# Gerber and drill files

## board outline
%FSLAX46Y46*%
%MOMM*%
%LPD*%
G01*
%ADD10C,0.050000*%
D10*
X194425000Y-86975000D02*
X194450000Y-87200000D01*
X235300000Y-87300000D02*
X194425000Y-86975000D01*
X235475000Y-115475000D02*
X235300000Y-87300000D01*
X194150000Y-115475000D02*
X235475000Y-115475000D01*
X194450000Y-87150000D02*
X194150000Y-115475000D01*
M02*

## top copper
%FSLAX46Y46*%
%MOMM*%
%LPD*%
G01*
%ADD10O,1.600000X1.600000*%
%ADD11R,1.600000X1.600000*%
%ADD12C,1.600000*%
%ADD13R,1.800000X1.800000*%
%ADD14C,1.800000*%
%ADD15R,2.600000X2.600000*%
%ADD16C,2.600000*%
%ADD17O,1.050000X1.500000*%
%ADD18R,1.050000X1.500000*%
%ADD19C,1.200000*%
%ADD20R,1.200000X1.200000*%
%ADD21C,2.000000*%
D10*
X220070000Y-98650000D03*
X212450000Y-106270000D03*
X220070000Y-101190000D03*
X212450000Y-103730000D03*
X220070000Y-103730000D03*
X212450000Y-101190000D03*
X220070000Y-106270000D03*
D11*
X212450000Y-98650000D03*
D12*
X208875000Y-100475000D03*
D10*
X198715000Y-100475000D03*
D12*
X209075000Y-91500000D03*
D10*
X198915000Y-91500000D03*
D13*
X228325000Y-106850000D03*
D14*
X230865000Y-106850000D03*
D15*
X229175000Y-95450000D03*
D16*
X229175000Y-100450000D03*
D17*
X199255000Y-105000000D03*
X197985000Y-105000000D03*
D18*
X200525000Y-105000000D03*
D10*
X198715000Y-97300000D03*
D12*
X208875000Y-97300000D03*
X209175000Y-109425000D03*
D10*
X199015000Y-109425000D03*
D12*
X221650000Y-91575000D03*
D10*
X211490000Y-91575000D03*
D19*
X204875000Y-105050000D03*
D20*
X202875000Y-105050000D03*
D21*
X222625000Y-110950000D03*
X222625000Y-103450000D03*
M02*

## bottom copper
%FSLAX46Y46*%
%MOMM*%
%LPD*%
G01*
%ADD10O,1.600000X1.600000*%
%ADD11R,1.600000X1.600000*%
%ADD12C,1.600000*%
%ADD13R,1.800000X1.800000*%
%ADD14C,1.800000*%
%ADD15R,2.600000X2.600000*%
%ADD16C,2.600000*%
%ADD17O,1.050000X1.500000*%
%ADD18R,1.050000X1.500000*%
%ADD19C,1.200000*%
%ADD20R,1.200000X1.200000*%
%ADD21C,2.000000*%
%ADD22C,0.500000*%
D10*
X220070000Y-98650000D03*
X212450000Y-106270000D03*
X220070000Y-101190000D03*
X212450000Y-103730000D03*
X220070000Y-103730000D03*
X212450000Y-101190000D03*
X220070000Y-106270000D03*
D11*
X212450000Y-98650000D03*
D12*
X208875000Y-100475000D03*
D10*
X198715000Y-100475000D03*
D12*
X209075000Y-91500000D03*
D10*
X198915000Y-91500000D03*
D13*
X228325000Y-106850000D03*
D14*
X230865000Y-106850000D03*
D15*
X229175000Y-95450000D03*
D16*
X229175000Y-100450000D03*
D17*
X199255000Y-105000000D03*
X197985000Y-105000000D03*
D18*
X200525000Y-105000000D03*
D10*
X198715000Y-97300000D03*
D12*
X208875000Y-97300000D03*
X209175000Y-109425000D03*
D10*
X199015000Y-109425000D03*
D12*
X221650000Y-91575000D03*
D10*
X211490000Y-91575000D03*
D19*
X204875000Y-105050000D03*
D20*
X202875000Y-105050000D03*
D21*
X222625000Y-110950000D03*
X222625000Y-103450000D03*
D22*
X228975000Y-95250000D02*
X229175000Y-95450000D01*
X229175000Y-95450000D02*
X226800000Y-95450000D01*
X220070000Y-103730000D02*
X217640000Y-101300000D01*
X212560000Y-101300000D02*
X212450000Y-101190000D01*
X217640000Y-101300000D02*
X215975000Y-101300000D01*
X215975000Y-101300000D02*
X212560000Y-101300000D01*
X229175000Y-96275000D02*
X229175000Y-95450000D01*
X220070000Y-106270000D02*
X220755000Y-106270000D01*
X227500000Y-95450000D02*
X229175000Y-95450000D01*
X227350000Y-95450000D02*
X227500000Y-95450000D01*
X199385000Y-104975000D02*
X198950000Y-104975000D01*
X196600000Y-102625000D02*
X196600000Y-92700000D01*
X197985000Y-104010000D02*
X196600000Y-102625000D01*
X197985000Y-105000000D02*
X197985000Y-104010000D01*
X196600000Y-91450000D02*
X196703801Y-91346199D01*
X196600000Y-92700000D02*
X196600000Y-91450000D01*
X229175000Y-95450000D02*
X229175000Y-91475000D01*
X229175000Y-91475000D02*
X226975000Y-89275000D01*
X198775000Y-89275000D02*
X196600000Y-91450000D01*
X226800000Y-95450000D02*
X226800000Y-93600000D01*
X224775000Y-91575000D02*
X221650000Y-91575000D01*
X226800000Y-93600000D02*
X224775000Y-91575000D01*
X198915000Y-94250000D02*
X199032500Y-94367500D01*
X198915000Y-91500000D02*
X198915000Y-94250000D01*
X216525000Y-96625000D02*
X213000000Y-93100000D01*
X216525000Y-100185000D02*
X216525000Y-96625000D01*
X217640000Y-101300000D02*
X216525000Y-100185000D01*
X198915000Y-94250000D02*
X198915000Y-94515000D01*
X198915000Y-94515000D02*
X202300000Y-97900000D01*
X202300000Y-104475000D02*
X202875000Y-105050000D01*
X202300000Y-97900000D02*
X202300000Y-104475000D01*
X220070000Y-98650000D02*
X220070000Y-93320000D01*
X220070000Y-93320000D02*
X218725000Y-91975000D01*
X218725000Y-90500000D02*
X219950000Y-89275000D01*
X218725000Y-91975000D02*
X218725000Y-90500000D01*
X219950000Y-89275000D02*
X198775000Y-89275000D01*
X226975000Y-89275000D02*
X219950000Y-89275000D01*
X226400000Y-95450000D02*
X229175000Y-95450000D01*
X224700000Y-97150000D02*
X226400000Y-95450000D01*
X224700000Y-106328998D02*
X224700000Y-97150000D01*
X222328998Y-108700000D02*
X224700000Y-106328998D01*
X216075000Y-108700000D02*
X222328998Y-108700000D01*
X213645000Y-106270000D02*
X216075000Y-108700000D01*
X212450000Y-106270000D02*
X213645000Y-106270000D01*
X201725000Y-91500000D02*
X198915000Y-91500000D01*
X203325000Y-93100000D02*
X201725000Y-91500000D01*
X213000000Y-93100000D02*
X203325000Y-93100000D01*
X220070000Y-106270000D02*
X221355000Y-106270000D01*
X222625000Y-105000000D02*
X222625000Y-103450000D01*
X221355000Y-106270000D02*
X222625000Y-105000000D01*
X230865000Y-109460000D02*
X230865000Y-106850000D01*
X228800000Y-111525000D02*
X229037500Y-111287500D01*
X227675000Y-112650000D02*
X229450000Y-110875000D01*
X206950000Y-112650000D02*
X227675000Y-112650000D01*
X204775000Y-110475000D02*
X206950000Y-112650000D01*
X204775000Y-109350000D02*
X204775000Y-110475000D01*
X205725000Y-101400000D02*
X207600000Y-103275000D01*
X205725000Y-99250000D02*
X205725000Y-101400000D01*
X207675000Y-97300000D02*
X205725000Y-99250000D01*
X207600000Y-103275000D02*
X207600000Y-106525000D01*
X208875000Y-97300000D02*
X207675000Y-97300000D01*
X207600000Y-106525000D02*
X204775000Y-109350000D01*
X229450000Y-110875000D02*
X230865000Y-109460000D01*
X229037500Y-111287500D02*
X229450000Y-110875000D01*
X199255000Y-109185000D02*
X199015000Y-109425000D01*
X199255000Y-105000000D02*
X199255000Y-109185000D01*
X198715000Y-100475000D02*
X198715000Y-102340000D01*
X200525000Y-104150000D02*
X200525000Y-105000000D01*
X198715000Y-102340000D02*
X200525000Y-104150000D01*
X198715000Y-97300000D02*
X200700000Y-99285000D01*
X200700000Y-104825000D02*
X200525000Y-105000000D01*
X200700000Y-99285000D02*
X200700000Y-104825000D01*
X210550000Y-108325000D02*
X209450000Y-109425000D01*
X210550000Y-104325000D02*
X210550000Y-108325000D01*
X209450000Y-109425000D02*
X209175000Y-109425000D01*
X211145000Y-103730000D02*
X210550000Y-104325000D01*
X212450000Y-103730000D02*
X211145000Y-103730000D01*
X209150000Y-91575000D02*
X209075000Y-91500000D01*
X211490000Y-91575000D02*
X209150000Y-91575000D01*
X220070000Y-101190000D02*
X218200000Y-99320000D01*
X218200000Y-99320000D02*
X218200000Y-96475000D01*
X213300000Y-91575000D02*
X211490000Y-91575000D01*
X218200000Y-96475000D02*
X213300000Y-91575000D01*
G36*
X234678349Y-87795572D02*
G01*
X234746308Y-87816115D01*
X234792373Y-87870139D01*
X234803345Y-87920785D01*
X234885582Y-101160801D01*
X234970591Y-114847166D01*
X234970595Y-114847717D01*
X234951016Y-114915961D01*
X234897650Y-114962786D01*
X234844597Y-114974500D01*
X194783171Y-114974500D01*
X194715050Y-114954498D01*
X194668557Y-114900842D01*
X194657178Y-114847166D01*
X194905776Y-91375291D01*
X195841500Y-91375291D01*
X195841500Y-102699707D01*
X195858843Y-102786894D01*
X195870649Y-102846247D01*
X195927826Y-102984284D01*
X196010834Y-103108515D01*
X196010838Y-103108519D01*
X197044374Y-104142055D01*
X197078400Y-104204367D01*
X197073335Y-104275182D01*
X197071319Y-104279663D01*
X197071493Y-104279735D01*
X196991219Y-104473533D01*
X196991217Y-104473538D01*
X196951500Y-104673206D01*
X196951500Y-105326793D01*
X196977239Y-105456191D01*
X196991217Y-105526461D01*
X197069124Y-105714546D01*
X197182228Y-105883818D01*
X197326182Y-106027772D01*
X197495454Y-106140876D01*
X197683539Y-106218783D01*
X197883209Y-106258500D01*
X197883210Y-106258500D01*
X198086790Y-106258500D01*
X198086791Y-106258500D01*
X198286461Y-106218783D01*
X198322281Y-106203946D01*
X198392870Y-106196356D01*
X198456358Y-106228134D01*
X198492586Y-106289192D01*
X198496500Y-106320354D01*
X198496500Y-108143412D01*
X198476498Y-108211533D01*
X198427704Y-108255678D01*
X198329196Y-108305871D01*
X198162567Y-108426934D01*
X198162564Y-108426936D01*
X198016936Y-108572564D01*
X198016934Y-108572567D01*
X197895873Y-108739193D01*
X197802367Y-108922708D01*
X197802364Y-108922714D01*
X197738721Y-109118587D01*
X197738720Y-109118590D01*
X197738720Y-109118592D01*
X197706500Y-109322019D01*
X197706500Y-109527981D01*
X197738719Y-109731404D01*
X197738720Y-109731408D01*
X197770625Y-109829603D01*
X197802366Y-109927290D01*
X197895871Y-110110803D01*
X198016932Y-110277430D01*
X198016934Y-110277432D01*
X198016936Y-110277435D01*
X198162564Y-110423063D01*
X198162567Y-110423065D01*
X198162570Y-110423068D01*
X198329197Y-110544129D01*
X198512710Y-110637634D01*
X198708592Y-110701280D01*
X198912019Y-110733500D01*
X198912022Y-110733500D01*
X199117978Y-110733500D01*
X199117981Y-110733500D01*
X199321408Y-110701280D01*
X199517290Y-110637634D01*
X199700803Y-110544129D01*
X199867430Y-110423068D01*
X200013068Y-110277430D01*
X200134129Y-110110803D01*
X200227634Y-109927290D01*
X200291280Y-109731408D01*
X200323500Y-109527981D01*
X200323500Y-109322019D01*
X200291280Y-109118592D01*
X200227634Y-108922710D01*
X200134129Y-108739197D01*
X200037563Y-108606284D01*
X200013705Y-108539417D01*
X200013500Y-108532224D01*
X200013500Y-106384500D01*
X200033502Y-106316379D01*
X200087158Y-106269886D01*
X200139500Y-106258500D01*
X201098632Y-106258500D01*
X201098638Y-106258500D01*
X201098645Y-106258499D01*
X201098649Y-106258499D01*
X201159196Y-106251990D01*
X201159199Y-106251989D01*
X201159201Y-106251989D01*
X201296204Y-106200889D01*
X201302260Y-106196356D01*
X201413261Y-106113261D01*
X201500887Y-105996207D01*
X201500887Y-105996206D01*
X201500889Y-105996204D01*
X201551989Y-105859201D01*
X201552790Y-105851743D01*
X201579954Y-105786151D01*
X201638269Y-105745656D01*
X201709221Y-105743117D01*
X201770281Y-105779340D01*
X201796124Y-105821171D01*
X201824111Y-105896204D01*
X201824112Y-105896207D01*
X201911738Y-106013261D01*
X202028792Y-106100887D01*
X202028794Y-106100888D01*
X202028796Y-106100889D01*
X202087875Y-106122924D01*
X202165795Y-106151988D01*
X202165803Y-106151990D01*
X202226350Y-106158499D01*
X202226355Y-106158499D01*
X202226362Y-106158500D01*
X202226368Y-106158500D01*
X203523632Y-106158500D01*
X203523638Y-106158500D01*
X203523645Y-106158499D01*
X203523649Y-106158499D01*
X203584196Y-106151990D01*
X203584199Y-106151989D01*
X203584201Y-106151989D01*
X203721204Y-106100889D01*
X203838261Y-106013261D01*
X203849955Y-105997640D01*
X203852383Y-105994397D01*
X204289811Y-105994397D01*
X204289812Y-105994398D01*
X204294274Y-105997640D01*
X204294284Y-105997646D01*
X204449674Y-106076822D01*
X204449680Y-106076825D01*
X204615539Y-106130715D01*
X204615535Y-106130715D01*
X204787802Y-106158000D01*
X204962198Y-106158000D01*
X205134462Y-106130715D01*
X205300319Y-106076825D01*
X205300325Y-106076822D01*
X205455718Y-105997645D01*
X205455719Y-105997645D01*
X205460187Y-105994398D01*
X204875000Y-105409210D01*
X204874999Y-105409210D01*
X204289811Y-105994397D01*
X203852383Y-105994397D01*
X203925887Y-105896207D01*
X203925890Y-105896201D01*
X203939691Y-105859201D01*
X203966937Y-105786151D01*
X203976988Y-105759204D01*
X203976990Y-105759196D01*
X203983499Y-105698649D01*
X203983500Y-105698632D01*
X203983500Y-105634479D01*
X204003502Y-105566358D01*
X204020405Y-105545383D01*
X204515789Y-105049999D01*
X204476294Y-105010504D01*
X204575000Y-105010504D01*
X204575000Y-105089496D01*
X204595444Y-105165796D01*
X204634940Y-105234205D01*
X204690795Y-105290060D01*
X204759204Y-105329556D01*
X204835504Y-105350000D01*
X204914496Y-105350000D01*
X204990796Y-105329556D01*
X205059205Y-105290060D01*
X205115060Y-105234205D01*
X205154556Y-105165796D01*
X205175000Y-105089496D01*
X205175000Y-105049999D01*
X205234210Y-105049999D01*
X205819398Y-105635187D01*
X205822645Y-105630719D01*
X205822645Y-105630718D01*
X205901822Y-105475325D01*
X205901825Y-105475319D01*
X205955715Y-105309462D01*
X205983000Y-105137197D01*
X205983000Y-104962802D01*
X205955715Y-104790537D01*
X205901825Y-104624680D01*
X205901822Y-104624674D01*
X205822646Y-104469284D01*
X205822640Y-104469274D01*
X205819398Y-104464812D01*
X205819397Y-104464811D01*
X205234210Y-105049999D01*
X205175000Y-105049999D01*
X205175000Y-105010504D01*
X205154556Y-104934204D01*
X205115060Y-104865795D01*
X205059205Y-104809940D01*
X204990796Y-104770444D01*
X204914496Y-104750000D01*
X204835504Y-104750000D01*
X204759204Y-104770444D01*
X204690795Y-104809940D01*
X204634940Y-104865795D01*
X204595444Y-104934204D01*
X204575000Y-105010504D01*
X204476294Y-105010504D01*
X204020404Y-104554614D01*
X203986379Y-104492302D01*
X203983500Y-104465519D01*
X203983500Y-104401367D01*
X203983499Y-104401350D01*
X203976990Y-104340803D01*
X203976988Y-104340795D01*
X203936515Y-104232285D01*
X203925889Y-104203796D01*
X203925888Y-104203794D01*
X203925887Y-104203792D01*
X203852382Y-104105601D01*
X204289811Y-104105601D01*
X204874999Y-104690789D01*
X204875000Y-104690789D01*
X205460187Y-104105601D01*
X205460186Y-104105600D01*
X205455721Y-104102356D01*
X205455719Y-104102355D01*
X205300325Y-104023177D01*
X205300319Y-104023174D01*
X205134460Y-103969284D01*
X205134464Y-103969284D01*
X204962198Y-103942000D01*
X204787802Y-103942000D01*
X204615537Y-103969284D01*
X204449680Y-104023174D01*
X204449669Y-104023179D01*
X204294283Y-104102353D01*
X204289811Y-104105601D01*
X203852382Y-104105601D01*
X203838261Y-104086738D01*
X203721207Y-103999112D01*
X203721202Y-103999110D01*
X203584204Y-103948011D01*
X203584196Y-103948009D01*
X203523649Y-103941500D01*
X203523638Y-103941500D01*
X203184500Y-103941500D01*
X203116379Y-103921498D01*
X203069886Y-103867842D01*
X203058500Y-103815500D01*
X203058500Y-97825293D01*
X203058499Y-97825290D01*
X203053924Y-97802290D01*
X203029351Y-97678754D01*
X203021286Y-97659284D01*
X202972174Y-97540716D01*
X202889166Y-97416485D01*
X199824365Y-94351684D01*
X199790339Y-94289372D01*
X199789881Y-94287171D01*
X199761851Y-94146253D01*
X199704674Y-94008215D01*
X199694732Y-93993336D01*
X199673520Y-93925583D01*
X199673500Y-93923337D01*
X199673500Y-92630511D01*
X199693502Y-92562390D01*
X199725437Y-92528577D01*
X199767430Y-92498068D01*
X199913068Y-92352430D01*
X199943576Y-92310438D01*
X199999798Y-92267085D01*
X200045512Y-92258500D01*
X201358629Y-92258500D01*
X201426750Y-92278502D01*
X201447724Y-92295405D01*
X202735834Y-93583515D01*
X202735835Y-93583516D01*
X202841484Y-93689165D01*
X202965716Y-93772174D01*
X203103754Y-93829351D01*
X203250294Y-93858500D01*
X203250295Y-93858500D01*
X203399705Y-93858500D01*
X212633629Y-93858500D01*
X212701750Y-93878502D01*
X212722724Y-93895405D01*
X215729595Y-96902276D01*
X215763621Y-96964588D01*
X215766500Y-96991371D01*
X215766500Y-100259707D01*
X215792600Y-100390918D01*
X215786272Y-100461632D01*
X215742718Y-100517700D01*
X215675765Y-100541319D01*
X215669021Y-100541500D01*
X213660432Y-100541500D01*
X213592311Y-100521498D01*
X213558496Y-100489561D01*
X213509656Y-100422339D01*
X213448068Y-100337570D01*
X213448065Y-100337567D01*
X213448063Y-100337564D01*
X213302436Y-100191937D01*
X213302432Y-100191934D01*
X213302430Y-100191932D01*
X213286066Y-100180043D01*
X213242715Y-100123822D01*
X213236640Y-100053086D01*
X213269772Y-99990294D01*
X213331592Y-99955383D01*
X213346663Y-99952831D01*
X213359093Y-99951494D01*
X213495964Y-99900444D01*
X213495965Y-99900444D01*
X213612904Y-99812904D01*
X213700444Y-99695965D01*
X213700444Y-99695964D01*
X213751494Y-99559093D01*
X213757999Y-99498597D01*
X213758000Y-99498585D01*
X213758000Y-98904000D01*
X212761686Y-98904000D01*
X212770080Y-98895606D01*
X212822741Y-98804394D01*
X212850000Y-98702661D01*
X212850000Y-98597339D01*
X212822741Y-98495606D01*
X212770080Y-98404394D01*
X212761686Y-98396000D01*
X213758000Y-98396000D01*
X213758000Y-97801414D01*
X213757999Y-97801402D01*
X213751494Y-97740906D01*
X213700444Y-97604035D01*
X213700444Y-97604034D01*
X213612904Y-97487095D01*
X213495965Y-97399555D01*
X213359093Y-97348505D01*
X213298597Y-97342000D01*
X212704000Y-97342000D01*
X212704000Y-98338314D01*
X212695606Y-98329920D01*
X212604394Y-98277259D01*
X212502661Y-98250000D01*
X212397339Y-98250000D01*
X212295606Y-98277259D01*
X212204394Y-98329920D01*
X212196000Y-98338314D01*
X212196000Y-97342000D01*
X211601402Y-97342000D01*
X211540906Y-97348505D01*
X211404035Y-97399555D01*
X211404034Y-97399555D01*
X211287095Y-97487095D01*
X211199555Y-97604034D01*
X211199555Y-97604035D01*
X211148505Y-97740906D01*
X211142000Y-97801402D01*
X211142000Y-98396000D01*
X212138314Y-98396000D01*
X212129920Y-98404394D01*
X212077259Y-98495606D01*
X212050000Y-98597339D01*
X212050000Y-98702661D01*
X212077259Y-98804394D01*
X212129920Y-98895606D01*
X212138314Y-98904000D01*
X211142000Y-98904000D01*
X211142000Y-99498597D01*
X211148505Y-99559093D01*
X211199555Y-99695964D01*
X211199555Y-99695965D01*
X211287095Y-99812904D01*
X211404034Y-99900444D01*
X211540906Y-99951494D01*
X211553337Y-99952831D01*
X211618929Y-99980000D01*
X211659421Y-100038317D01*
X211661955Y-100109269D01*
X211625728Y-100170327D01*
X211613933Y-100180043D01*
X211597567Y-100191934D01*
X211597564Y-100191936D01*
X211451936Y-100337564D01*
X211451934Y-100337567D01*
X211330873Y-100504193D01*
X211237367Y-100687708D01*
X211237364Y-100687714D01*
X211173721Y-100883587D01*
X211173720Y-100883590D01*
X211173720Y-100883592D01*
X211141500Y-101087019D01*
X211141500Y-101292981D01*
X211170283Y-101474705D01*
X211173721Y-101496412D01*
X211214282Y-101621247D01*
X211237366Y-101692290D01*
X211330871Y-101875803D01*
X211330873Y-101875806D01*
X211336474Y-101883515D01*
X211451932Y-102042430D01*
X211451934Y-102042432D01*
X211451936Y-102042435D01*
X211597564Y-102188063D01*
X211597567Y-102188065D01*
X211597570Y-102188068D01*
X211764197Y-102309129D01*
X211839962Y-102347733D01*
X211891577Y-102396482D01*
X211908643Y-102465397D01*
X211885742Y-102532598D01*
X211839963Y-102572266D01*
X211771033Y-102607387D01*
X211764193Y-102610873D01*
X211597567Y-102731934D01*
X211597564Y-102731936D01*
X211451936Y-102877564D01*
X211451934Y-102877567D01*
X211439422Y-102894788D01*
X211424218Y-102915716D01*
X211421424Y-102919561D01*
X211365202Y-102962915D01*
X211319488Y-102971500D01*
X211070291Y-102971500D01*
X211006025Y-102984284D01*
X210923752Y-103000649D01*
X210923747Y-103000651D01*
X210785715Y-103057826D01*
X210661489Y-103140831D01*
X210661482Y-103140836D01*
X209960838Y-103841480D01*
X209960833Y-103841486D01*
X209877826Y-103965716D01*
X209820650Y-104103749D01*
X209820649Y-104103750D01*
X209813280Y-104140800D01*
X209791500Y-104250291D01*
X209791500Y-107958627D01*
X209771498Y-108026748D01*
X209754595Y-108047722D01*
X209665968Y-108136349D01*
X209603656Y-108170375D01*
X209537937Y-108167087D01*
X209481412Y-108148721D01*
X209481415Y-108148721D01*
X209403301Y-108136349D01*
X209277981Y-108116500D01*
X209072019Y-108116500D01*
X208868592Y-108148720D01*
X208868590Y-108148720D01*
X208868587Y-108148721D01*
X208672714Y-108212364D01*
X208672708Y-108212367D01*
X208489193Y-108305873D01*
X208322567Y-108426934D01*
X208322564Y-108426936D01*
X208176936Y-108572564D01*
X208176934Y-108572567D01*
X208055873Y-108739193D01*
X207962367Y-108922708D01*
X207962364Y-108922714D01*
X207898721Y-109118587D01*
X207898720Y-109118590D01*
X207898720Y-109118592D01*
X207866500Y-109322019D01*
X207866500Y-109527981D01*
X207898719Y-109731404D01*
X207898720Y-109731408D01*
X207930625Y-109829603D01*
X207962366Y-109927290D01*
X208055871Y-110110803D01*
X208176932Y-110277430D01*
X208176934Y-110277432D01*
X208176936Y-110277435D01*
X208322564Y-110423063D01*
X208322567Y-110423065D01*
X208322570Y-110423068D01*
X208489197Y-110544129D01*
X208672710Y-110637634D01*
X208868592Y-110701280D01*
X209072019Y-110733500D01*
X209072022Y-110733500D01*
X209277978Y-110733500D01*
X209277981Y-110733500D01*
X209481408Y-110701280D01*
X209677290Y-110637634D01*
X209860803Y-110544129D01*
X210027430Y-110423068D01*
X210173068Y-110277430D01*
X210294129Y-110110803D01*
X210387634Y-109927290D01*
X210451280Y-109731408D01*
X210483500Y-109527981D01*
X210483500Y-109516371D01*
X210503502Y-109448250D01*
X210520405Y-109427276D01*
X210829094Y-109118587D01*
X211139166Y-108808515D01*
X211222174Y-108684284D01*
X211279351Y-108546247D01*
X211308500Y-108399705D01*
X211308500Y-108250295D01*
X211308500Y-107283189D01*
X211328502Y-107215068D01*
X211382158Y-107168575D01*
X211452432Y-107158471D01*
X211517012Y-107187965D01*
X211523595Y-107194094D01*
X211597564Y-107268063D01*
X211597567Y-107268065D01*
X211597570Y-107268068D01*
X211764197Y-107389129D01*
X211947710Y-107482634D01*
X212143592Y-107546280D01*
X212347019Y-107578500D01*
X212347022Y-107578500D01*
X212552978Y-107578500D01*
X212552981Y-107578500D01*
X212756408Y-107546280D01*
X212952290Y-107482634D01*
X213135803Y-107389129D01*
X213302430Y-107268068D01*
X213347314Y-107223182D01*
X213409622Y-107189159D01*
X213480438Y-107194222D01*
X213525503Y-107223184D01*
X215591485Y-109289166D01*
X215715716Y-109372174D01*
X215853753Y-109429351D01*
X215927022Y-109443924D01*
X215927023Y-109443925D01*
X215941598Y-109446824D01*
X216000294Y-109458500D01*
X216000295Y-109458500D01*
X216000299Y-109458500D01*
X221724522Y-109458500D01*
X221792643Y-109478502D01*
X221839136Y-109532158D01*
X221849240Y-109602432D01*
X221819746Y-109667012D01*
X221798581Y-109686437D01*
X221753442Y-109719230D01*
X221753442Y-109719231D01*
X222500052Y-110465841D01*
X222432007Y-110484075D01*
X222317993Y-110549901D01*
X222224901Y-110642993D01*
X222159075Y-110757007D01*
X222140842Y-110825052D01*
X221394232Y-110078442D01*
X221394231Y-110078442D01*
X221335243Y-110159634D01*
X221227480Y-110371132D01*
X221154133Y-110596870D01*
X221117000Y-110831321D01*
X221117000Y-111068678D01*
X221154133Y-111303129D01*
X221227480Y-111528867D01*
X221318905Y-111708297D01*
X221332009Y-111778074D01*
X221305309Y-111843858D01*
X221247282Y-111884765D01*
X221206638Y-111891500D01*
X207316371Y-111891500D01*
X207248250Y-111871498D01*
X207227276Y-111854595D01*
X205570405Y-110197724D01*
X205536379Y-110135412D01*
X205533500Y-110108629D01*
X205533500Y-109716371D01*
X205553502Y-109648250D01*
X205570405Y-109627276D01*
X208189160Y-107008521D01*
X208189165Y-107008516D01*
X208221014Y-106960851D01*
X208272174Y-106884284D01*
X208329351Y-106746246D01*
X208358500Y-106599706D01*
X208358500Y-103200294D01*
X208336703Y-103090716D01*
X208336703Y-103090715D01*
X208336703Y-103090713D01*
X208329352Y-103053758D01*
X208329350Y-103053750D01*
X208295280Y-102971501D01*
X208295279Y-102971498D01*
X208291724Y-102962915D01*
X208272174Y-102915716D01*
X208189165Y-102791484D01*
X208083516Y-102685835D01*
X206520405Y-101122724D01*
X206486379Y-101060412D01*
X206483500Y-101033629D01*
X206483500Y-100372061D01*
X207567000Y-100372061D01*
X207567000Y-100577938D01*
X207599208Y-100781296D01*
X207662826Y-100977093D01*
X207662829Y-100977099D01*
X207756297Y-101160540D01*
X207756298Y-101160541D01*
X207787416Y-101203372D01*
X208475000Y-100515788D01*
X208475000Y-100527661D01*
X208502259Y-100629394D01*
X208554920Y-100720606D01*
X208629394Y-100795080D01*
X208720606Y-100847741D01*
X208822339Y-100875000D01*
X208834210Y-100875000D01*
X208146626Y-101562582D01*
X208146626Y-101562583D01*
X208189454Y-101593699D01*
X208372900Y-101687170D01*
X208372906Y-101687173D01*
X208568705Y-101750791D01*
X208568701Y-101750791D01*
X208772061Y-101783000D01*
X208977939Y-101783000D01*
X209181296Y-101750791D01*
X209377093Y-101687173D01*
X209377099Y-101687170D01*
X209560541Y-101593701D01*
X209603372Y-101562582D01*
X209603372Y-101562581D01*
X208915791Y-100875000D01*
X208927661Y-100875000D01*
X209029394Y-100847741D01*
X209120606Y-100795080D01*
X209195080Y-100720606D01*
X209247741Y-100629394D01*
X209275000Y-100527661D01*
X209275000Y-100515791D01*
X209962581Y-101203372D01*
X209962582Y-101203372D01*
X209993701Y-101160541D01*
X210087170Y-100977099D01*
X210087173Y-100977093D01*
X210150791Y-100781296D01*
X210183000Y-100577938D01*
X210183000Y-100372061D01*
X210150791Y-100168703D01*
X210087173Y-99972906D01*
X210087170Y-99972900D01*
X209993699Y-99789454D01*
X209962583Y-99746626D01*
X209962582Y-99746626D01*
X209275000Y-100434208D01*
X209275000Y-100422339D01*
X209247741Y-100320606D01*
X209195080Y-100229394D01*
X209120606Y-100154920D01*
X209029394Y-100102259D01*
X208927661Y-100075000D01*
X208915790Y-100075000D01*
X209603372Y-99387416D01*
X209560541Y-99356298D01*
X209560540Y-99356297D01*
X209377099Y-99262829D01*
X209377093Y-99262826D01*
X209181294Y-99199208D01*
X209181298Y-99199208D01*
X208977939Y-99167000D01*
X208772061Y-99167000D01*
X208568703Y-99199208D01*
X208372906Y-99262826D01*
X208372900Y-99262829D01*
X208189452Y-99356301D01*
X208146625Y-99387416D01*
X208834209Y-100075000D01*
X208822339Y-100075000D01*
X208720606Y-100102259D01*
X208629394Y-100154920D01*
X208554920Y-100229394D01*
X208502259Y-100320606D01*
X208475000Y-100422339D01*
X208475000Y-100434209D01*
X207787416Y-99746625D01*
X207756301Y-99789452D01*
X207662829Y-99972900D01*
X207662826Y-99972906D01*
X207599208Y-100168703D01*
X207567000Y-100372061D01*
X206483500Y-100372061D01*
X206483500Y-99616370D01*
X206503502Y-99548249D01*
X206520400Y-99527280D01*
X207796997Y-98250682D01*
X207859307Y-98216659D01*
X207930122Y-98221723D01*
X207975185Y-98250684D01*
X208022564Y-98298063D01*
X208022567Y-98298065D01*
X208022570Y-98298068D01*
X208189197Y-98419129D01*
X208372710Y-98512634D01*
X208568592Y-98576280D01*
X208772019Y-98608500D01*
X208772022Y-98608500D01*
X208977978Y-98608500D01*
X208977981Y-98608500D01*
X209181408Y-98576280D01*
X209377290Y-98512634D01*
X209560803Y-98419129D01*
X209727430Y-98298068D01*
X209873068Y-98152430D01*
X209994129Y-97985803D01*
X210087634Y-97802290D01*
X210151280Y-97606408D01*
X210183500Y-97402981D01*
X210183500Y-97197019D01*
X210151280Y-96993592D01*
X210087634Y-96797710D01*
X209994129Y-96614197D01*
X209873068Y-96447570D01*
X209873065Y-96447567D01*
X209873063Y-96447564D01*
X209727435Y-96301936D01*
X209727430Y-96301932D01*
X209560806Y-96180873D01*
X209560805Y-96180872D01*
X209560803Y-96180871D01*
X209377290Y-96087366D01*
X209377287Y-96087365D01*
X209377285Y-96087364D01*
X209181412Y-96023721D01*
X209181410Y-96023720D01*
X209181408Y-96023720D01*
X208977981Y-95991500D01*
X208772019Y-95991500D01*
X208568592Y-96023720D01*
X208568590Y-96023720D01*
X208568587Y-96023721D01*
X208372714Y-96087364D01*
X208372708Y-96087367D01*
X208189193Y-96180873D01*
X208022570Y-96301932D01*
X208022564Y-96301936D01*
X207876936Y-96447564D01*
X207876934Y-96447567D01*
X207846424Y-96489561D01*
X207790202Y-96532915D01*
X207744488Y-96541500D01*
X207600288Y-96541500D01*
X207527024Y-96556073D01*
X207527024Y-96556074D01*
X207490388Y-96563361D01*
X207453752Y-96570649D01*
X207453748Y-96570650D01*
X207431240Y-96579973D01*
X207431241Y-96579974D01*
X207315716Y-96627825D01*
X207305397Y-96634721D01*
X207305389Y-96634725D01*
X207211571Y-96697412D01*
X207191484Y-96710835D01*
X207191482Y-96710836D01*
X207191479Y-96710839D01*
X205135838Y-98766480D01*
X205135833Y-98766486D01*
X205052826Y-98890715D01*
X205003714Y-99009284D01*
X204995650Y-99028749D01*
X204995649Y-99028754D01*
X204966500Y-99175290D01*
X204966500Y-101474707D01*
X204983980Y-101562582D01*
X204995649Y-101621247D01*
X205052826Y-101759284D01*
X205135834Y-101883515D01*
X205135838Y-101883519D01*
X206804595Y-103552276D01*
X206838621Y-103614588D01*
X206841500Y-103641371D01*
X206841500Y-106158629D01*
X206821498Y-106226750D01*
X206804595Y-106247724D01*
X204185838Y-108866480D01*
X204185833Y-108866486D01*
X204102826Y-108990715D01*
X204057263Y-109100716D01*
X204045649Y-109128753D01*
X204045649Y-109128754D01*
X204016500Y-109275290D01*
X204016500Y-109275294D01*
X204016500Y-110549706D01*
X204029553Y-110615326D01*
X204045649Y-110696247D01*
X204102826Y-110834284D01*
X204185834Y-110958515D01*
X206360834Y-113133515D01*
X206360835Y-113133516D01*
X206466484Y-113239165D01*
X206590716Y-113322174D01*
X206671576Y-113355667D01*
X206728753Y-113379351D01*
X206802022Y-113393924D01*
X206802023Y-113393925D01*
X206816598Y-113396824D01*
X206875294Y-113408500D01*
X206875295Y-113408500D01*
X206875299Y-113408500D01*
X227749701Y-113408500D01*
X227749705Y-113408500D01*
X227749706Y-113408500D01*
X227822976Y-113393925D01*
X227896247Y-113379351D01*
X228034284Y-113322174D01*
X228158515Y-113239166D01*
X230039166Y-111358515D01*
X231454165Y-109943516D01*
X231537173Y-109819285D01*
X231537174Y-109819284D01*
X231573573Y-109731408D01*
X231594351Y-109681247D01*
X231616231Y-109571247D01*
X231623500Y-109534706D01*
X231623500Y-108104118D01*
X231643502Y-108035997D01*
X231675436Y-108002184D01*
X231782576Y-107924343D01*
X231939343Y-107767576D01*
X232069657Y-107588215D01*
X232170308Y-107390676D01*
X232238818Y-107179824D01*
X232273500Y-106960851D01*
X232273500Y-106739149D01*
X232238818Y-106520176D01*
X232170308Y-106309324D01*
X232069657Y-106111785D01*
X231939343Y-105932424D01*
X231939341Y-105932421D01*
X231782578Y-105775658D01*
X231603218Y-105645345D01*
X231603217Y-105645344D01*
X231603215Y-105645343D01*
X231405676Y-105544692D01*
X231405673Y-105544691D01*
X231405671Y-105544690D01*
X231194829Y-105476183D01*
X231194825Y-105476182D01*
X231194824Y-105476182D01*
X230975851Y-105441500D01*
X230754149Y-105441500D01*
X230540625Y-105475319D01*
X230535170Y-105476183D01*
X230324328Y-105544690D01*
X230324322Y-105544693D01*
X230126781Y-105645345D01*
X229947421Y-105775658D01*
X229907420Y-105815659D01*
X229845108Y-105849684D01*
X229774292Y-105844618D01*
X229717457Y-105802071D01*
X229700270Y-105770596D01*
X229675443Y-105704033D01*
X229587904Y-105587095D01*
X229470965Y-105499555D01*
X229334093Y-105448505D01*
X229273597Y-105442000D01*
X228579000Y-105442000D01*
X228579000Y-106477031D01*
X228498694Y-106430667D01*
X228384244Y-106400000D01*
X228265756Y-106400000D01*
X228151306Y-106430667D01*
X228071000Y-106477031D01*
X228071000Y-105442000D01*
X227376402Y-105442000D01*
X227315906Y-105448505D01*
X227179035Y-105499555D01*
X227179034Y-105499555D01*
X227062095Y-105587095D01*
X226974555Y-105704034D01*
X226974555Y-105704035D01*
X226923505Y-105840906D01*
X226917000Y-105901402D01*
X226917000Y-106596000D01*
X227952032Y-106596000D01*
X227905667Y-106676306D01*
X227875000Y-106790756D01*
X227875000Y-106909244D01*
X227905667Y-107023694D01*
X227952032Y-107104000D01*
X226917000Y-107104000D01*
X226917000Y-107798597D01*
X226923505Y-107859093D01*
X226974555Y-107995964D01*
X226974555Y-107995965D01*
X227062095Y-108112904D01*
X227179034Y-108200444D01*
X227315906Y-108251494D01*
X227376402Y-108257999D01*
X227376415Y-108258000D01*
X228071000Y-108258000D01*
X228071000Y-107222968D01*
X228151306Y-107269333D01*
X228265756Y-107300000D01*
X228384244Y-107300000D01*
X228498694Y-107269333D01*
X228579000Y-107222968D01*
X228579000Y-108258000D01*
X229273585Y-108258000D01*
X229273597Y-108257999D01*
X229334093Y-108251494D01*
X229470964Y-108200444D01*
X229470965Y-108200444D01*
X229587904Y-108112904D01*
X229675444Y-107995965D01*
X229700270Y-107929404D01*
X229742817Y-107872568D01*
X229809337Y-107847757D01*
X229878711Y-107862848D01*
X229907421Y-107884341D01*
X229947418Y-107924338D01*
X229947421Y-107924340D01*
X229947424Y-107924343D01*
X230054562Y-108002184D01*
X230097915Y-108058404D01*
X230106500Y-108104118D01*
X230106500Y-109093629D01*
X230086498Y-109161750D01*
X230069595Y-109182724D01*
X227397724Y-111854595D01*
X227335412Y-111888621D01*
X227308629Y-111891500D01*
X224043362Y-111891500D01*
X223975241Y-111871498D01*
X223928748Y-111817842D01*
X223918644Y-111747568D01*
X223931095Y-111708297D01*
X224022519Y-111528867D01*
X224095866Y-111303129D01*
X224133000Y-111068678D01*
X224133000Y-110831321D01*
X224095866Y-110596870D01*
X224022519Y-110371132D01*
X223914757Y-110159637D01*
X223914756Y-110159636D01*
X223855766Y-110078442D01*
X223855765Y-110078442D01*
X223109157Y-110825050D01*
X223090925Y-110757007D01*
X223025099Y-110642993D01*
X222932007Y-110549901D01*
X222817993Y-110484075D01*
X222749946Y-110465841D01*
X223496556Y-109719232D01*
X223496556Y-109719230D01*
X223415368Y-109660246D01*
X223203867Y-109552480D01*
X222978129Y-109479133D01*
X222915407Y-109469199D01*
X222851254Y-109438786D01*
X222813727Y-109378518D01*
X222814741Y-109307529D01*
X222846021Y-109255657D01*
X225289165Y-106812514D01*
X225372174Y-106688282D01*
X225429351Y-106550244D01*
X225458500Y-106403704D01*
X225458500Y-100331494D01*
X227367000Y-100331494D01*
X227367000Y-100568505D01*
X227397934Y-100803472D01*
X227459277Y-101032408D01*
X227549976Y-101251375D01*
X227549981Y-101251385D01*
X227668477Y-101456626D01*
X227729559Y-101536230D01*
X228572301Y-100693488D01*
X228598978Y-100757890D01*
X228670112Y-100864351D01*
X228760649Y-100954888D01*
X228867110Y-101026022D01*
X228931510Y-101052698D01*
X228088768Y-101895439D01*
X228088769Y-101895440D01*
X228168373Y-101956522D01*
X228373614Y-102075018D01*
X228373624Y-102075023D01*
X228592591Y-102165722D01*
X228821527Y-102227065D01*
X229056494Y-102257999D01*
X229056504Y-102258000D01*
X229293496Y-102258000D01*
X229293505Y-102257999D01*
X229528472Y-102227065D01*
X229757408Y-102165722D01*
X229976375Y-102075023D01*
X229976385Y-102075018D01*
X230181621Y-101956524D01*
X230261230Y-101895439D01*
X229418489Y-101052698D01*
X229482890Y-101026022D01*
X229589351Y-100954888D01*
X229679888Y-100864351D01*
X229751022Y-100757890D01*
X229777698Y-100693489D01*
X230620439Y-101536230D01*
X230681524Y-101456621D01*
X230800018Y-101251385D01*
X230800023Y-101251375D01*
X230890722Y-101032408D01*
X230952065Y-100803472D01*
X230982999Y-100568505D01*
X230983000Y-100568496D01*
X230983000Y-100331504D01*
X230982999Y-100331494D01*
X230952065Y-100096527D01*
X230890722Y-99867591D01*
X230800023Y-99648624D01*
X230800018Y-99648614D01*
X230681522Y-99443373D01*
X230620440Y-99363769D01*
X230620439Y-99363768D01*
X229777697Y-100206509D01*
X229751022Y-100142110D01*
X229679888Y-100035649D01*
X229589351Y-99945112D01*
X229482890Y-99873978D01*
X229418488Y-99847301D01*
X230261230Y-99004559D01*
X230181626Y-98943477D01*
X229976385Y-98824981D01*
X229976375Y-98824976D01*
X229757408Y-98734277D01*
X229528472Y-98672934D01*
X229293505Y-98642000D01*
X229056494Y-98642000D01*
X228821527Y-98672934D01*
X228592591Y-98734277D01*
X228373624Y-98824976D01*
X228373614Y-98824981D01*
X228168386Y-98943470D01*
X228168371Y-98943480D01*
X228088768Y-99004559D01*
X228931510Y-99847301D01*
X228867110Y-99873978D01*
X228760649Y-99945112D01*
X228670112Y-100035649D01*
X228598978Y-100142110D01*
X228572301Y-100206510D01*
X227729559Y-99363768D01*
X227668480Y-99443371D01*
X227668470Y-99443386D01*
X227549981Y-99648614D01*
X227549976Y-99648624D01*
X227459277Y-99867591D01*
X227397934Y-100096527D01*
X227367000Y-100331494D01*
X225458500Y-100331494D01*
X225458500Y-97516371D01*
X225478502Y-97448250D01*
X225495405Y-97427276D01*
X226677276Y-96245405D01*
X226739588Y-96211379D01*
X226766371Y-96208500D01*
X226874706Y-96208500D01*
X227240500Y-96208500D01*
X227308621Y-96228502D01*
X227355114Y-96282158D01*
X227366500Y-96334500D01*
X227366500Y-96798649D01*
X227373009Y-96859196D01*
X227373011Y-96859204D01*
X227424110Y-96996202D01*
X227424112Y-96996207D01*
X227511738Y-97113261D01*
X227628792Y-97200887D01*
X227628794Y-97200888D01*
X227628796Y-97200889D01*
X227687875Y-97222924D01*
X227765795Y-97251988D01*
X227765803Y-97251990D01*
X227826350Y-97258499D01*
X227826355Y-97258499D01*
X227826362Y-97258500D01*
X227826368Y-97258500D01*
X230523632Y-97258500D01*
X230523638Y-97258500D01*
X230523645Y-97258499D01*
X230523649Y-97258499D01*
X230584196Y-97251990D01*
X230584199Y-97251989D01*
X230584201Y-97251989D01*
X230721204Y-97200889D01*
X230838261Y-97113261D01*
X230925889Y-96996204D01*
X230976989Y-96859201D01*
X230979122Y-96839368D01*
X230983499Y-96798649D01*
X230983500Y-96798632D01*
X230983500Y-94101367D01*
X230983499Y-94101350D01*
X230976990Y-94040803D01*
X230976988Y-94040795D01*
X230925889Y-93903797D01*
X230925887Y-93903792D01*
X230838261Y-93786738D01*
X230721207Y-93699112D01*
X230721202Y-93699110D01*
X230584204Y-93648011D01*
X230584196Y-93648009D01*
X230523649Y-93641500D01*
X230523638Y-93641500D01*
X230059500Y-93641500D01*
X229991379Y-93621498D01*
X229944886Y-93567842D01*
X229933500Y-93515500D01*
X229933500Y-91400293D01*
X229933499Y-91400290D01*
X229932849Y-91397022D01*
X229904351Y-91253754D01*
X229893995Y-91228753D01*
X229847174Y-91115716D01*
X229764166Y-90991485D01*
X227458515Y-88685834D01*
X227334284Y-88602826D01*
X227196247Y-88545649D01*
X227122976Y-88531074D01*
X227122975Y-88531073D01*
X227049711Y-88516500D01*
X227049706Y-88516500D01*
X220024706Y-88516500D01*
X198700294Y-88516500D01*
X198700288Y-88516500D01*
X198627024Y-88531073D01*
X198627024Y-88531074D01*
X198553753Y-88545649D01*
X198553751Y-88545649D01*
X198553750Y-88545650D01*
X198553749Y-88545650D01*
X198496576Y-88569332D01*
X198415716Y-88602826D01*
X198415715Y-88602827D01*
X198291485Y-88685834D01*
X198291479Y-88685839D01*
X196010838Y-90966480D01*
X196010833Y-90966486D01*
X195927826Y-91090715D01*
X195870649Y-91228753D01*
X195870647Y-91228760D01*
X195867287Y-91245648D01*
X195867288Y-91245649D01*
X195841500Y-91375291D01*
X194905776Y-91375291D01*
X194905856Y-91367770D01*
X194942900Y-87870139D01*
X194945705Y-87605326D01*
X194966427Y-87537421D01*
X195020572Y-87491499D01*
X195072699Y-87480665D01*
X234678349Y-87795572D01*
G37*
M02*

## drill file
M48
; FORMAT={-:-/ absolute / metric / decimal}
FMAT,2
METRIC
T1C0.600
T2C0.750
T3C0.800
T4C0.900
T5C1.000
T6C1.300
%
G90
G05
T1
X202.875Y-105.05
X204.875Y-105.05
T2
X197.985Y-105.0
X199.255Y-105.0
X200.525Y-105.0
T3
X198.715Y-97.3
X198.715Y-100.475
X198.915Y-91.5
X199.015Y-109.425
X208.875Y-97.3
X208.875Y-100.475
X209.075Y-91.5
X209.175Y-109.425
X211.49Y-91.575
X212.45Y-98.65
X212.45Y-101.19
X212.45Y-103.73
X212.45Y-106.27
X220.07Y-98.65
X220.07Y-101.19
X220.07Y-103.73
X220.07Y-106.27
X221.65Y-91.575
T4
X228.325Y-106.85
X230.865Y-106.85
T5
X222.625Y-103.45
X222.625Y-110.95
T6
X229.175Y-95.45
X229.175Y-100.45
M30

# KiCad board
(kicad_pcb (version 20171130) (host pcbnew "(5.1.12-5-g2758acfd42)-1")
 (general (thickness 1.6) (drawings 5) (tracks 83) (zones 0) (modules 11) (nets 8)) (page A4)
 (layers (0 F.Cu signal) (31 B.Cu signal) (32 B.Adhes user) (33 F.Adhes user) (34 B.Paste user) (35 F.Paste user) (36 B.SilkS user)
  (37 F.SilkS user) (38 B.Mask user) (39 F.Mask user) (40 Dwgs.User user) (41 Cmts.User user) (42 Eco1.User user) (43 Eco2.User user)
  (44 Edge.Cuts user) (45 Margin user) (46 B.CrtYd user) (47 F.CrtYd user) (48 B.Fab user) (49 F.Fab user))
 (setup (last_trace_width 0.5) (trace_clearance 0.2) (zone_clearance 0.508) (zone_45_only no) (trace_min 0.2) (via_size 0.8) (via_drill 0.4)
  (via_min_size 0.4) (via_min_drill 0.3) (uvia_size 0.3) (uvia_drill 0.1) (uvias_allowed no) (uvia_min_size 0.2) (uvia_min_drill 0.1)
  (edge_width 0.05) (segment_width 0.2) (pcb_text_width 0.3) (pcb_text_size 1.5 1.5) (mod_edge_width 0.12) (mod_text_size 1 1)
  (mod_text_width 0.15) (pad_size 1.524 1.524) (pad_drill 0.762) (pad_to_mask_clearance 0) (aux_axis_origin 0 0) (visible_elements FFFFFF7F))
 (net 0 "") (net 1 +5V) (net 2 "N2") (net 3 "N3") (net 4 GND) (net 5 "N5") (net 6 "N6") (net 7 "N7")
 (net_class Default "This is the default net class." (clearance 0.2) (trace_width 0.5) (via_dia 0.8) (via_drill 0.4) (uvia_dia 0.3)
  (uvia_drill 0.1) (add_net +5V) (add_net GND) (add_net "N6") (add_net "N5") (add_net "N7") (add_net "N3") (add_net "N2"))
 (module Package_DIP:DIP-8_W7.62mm (layer F.Cu) (at 212.45 98.65)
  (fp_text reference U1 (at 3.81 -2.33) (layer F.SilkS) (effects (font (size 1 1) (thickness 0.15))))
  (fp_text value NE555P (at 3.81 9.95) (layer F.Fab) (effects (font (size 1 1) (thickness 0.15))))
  (pad 8 thru_hole oval (at 7.62 0) (size 1.6 1.6) (drill 0.8) (layers *.Cu *.Mask) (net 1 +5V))
  (pad 4 thru_hole oval (at 0 7.62) (size 1.6 1.6) (drill 0.8) (layers *.Cu *.Mask) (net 1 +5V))
  (pad 7 thru_hole oval (at 7.62 2.54) (size 1.6 1.6) (drill 0.8) (layers *.Cu *.Mask) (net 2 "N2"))
  (pad 3 thru_hole oval (at 0 5.08) (size 1.6 1.6) (drill 0.8) (layers *.Cu *.Mask) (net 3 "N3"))
  (pad 6 thru_hole oval (at 7.62 5.08) (size 1.6 1.6) (drill 0.8) (layers *.Cu *.Mask) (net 1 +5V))
  (pad 2 thru_hole oval (at 0 2.54) (size 1.6 1.6) (drill 0.8) (layers *.Cu *.Mask) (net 1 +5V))
  (pad 5 thru_hole oval (at 7.62 7.62) (size 1.6 1.6) (drill 0.8) (layers *.Cu *.Mask) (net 1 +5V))
  (pad 1 thru_hole rect (at 0 0) (size 1.6 1.6) (drill 0.8) (layers *.Cu *.Mask) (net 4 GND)))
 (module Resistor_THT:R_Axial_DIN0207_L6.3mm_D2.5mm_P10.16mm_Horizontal (layer F.Cu) (at 208.875 100.475 180)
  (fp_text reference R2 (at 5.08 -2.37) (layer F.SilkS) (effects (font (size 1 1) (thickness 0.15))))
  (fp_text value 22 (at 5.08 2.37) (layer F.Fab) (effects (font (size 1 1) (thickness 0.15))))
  (pad 1 thru_hole circle (at 0 0 180) (size 1.6 1.6) (drill 0.8) (layers *.Cu *.Mask) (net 4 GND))
  (pad 2 thru_hole oval (at 10.16 0 180) (size 1.6 1.6) (drill 0.8) (layers *.Cu *.Mask) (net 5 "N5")))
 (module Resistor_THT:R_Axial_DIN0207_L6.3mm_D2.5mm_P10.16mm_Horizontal (layer F.Cu) (at 209.075 91.5 180)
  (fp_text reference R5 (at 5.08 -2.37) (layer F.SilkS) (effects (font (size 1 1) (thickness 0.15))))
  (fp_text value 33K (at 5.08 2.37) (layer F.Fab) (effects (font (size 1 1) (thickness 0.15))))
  (pad 1 thru_hole circle (at 0 0 180) (size 1.6 1.6) (drill 0.8) (layers *.Cu *.Mask) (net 2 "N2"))
  (pad 2 thru_hole oval (at 10.16 0 180) (size 1.6 1.6) (drill 0.8) (layers *.Cu *.Mask) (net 1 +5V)))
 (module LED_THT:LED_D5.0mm (layer F.Cu) (at 228.325 106.85)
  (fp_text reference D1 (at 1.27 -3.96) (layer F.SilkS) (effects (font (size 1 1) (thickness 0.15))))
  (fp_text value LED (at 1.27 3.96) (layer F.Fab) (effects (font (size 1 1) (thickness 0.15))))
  (pad 1 thru_hole rect (at 0 0) (size 1.8 1.8) (drill 0.9) (layers *.Cu *.Mask) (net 4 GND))
  (pad 2 thru_hole circle (at 2.54 0) (size 1.8 1.8) (drill 0.9) (layers *.Cu *.Mask) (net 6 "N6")))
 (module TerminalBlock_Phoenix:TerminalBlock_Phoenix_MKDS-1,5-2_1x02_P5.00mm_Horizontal (layer F.Cu) (at 229.175 95.45 270)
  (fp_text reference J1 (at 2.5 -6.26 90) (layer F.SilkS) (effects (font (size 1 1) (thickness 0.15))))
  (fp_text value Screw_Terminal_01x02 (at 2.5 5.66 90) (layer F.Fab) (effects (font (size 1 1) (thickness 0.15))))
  (pad 1 thru_hole rect (at 0 0 270) (size 2.6 2.6) (drill 1.3) (layers *.Cu *.Mask) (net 1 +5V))
  (pad 2 thru_hole circle (at 5 0 270) (size 2.6 2.6) (drill 1.3) (layers *.Cu *.Mask) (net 4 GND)))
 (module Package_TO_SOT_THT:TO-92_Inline (layer F.Cu) (at 200.525 105 180)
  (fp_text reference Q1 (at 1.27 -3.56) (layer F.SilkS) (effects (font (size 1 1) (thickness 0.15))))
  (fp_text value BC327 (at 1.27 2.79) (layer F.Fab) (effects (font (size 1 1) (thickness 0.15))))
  (pad 2 thru_hole oval (at 1.27 0 180) (size 1.05 1.5) (drill 0.75) (layers *.Cu *.Mask) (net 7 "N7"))
  (pad 3 thru_hole oval (at 2.54 0 180) (size 1.05 1.5) (drill 0.75) (layers *.Cu *.Mask) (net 1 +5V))
  (pad 1 thru_hole rect (at 0 0 180) (size 1.05 1.5) (drill 0.75) (layers *.Cu *.Mask) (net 5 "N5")))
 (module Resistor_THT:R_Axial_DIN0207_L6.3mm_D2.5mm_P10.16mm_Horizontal (layer F.Cu) (at 208.875 97.3 180)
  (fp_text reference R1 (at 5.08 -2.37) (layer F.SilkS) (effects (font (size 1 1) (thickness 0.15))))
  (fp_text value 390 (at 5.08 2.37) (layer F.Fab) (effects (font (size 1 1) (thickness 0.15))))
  (pad 2 thru_hole oval (at 10.16 0 180) (size 1.6 1.6) (drill 0.8) (layers *.Cu *.Mask) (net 5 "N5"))
  (pad 1 thru_hole circle (at 0 0 180) (size 1.6 1.6) (drill 0.8) (layers *.Cu *.Mask) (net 6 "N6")))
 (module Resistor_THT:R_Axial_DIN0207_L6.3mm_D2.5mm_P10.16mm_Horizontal (layer F.Cu) (at 209.175 109.425 180)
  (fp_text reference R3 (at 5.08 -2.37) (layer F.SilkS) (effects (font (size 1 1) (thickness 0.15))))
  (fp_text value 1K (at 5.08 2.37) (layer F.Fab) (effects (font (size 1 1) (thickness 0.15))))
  (pad 1 thru_hole circle (at 0 0 180) (size 1.6 1.6) (drill 0.8) (layers *.Cu *.Mask) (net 3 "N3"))
  (pad 2 thru_hole oval (at 10.16 0 180) (size 1.6 1.6) (drill 0.8) (layers *.Cu *.Mask) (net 7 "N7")))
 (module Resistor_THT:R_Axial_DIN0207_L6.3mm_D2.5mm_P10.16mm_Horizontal (layer F.Cu) (at 221.65 91.575 180)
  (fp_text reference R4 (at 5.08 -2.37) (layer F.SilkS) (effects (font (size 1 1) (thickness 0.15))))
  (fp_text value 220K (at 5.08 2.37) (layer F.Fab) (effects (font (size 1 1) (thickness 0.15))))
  (pad 1 thru_hole circle (at 0 0 180) (size 1.6 1.6) (drill 0.8) (layers *.Cu *.Mask) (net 1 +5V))
  (pad 2 thru_hole oval (at 10.16 0 180) (size 1.6 1.6) (drill 0.8) (layers *.Cu *.Mask) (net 2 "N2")))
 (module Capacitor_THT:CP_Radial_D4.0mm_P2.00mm (layer F.Cu) (at 202.875 105.05)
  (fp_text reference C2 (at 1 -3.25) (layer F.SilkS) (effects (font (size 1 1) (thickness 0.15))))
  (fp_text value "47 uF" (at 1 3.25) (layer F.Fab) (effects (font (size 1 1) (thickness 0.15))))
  (pad 2 thru_hole circle (at 2 0) (size 1.2 1.2) (drill 0.6) (layers *.Cu *.Mask) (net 4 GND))
  (pad 1 thru_hole rect (at 0 0) (size 1.2 1.2) (drill 0.6) (layers *.Cu *.Mask) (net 1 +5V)))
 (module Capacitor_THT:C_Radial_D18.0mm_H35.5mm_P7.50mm (layer F.Cu) (at 222.625 110.95 90)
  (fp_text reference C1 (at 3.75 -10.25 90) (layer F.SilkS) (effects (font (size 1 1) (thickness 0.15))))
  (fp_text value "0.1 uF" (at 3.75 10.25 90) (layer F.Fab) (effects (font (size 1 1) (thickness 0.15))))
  (pad 1 thru_hole circle (at 0 0 90) (size 2 2) (drill 1) (layers *.Cu *.Mask) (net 4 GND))
  (pad 2 thru_hole circle (at 7.5 0 90) (size 2 2) (drill 1) (layers *.Cu *.Mask) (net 1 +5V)))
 (gr_line (start 194.425 86.975) (end 194.45 87.2) (layer Edge.Cuts) (width 0.05))
 (gr_line (start 235.3 87.3) (end 194.425 86.975) (layer Edge.Cuts) (width 0.05))
 (gr_line (start 235.475 115.475) (end 235.3 87.3) (layer Edge.Cuts) (width 0.05))
 (gr_line (start 194.15 115.475) (end 235.475 115.475) (layer Edge.Cuts) (width 0.05))
 (gr_line (start 194.45 87.15) (end 194.15 115.475) (layer Edge.Cuts) (width 0.05))
 (segment (start 228.975 95.25) (end 229.175 95.45) (width 0.5) (layer B.Cu) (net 1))
 (segment (start 229.175 95.45) (end 226.8 95.45) (width 0.5) (layer B.Cu) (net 1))
 (segment (start 220.07 103.73) (end 217.64 101.3) (width 0.5) (layer B.Cu) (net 1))
 (segment (start 212.56 101.3) (end 212.45 101.19) (width 0.5) (layer B.Cu) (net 1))
 (segment (start 217.64 101.3) (end 215.975 101.3) (width 0.5) (layer B.Cu) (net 1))
 (segment (start 215.975 101.3) (end 212.56 101.3) (width 0.5) (layer B.Cu) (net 1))
 (segment (start 229.175 96.275) (end 229.175 95.45) (width 0.5) (layer B.Cu) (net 1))
 (segment (start 220.07 106.27) (end 220.755 106.27) (width 0.5) (layer B.Cu) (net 1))
 (segment (start 227.5 95.45) (end 229.175 95.45) (width 0.5) (layer B.Cu) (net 1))
 (segment (start 227.35 95.45) (end 227.5 95.45) (width 0.5) (layer B.Cu) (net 1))
 (segment (start 199.385 104.975) (end 198.95 104.975) (width 0.5) (layer B.Cu) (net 7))
 (segment (start 196.6 102.625) (end 196.6 92.7) (width 0.5) (layer B.Cu) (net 1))
 (segment (start 197.985 104.01) (end 196.6 102.625) (width 0.5) (layer B.Cu) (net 1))
 (segment (start 197.985 105) (end 197.985 104.01) (width 0.5) (layer B.Cu) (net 1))
 (segment (start 196.6 91.45) (end 196.703801 91.346199) (width 0.5) (layer B.Cu) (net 1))
 (segment (start 196.6 92.7) (end 196.6 91.45) (width 0.5) (layer B.Cu) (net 1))
 (segment (start 229.175 95.45) (end 229.175 91.475) (width 0.5) (layer B.Cu) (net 1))
 (segment (start 229.175 91.475) (end 226.975 89.275) (width 0.5) (layer B.Cu) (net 1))
 (segment (start 198.775 89.275) (end 196.6 91.45) (width 0.5) (layer B.Cu) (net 1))
 (segment (start 226.8 95.45) (end 226.8 93.6) (width 0.5) (layer B.Cu) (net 1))
 (segment (start 224.775 91.575) (end 221.65 91.575) (width 0.5) (layer B.Cu) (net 1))
 (segment (start 226.8 93.6) (end 224.775 91.575) (width 0.5) (layer B.Cu) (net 1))
 (segment (start 198.915 94.25) (end 199.0325 94.3675) (width 0.5) (layer B.Cu) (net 1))
 (segment (start 198.915 91.5) (end 198.915 94.25) (width 0.5) (layer B.Cu) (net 1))
 (segment (start 216.525 96.625) (end 213 93.1) (width 0.5) (layer B.Cu) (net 1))
 (segment (start 216.525 100.185) (end 216.525 96.625) (width 0.5) (layer B.Cu) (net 1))
 (segment (start 217.64 101.3) (end 216.525 100.185) (width 0.5) (layer B.Cu) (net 1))
 (segment (start 198.915 94.25) (end 198.915 94.515) (width 0.5) (layer B.Cu) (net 1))
 (segment (start 198.915 94.515) (end 202.3 97.9) (width 0.5) (layer B.Cu) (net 1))
 (segment (start 202.3 104.475) (end 202.875 105.05) (width 0.5) (layer B.Cu) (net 1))
 (segment (start 202.3 97.9) (end 202.3 104.475) (width 0.5) (layer B.Cu) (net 1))
 (segment (start 220.07 98.65) (end 220.07 93.32) (width 0.5) (layer B.Cu) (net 1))
 (segment (start 220.07 93.32) (end 218.725 91.975) (width 0.5) (layer B.Cu) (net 1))
 (segment (start 218.725 90.5) (end 219.95 89.275) (width 0.5) (layer B.Cu) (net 1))
 (segment (start 218.725 91.975) (end 218.725 90.5) (width 0.5) (layer B.Cu) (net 1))
 (segment (start 219.95 89.275) (end 198.775 89.275) (width 0.5) (layer B.Cu) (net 1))
 (segment (start 226.975 89.275) (end 219.95 89.275) (width 0.5) (layer B.Cu) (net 1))
 (segment (start 226.4 95.45) (end 229.175 95.45) (width 0.5) (layer B.Cu) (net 1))
 (segment (start 224.7 97.15) (end 226.4 95.45) (width 0.5) (layer B.Cu) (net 1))
 (segment (start 224.7 106.328998) (end 224.7 97.15) (width 0.5) (layer B.Cu) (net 1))
 (segment (start 222.328998 108.7) (end 224.7 106.328998) (width 0.5) (layer B.Cu) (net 1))
 (segment (start 216.075 108.7) (end 222.328998 108.7) (width 0.5) (layer B.Cu) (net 1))
 (segment (start 213.645 106.27) (end 216.075 108.7) (width 0.5) (layer B.Cu) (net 1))
 (segment (start 212.45 106.27) (end 213.645 106.27) (width 0.5) (layer B.Cu) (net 1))
 (segment (start 201.725 91.5) (end 198.915 91.5) (width 0.5) (layer B.Cu) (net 1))
 (segment (start 203.325 93.1) (end 201.725 91.5) (width 0.5) (layer B.Cu) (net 1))
 (segment (start 213 93.1) (end 203.325 93.1) (width 0.5) (layer B.Cu) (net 1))
 (segment (start 220.07 106.27) (end 221.355 106.27) (width 0.5) (layer B.Cu) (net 1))
 (segment (start 222.625 105) (end 222.625 103.45) (width 0.5) (layer B.Cu) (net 1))
 (segment (start 221.355 106.27) (end 222.625 105) (width 0.5) (layer B.Cu) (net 1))
 (segment (start 230.865 109.46) (end 230.865 106.85) (width 0.5) (layer B.Cu) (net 6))
 (segment (start 228.8 111.525) (end 229.0375 111.2875) (width 0.5) (layer B.Cu) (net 6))
 (segment (start 227.675 112.65) (end 229.45 110.875) (width 0.5) (layer B.Cu) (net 6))
 (segment (start 206.95 112.65) (end 227.675 112.65) (width 0.5) (layer B.Cu) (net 6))
 (segment (start 204.775 110.475) (end 206.95 112.65) (width 0.5) (layer B.Cu) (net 6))
 (segment (start 204.775 109.35) (end 204.775 110.475) (width 0.5) (layer B.Cu) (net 6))
 (segment (start 205.725 101.4) (end 207.6 103.275) (width 0.5) (layer B.Cu) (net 6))
 (segment (start 205.725 99.25) (end 205.725 101.4) (width 0.5) (layer B.Cu) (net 6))
 (segment (start 207.675 97.3) (end 205.725 99.25) (width 0.5) (layer B.Cu) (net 6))
 (segment (start 207.6 103.275) (end 207.6 106.525) (width 0.5) (layer B.Cu) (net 6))
 (segment (start 208.875 97.3) (end 207.675 97.3) (width 0.5) (layer B.Cu) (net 6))
 (segment (start 207.6 106.525) (end 204.775 109.35) (width 0.5) (layer B.Cu) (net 6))
 (segment (start 229.45 110.875) (end 230.865 109.46) (width 0.5) (layer B.Cu) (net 6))
 (segment (start 229.0375 111.2875) (end 229.45 110.875) (width 0.5) (layer B.Cu) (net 6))
 (segment (start 199.255 109.185) (end 199.015 109.425) (width 0.5) (layer B.Cu) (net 7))
 (segment (start 199.255 105) (end 199.255 109.185) (width 0.5) (layer B.Cu) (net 7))
 (segment (start 198.715 100.475) (end 198.715 102.34) (width 0.5) (layer B.Cu) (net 5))
 (segment (start 200.525 104.15) (end 200.525 105) (width 0.5) (layer B.Cu) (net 5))
 (segment (start 198.715 102.34) (end 200.525 104.15) (width 0.5) (layer B.Cu) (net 5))
 (segment (start 198.715 97.3) (end 200.7 99.285) (width 0.5) (layer B.Cu) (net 5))
 (segment (start 200.7 104.825) (end 200.525 105) (width 0.5) (layer B.Cu) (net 5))
 (segment (start 200.7 99.285) (end 200.7 104.825) (width 0.5) (layer B.Cu) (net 5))
 (segment (start 210.55 108.325) (end 209.45 109.425) (width 0.5) (layer B.Cu) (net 3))
 (segment (start 210.55 104.325) (end 210.55 108.325) (width 0.5) (layer B.Cu) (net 3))
 (segment (start 209.45 109.425) (end 209.175 109.425) (width 0.5) (layer B.Cu) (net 3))
 (segment (start 211.145 103.73) (end 210.55 104.325) (width 0.5) (layer B.Cu) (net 3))
 (segment (start 212.45 103.73) (end 211.145 103.73) (width 0.5) (layer B.Cu) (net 3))
 (segment (start 209.15 91.575) (end 209.075 91.5) (width 0.5) (layer B.Cu) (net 2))
 (segment (start 211.49 91.575) (end 209.15 91.575) (width 0.5) (layer B.Cu) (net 2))
 (segment (start 220.07 101.19) (end 218.2 99.32) (width 0.5) (layer B.Cu) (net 2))
 (segment (start 218.2 99.32) (end 218.2 96.475) (width 0.5) (layer B.Cu) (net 2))
 (segment (start 213.3 91.575) (end 211.49 91.575) (width 0.5) (layer B.Cu) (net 2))
 (segment (start 218.2 96.475) (end 213.3 91.575) (width 0.5) (layer B.Cu) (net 2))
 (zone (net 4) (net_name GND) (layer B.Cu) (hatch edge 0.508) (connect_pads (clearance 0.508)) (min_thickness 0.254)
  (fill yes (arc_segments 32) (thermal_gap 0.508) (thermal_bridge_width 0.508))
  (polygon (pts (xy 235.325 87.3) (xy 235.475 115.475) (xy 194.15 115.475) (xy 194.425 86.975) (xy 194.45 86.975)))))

